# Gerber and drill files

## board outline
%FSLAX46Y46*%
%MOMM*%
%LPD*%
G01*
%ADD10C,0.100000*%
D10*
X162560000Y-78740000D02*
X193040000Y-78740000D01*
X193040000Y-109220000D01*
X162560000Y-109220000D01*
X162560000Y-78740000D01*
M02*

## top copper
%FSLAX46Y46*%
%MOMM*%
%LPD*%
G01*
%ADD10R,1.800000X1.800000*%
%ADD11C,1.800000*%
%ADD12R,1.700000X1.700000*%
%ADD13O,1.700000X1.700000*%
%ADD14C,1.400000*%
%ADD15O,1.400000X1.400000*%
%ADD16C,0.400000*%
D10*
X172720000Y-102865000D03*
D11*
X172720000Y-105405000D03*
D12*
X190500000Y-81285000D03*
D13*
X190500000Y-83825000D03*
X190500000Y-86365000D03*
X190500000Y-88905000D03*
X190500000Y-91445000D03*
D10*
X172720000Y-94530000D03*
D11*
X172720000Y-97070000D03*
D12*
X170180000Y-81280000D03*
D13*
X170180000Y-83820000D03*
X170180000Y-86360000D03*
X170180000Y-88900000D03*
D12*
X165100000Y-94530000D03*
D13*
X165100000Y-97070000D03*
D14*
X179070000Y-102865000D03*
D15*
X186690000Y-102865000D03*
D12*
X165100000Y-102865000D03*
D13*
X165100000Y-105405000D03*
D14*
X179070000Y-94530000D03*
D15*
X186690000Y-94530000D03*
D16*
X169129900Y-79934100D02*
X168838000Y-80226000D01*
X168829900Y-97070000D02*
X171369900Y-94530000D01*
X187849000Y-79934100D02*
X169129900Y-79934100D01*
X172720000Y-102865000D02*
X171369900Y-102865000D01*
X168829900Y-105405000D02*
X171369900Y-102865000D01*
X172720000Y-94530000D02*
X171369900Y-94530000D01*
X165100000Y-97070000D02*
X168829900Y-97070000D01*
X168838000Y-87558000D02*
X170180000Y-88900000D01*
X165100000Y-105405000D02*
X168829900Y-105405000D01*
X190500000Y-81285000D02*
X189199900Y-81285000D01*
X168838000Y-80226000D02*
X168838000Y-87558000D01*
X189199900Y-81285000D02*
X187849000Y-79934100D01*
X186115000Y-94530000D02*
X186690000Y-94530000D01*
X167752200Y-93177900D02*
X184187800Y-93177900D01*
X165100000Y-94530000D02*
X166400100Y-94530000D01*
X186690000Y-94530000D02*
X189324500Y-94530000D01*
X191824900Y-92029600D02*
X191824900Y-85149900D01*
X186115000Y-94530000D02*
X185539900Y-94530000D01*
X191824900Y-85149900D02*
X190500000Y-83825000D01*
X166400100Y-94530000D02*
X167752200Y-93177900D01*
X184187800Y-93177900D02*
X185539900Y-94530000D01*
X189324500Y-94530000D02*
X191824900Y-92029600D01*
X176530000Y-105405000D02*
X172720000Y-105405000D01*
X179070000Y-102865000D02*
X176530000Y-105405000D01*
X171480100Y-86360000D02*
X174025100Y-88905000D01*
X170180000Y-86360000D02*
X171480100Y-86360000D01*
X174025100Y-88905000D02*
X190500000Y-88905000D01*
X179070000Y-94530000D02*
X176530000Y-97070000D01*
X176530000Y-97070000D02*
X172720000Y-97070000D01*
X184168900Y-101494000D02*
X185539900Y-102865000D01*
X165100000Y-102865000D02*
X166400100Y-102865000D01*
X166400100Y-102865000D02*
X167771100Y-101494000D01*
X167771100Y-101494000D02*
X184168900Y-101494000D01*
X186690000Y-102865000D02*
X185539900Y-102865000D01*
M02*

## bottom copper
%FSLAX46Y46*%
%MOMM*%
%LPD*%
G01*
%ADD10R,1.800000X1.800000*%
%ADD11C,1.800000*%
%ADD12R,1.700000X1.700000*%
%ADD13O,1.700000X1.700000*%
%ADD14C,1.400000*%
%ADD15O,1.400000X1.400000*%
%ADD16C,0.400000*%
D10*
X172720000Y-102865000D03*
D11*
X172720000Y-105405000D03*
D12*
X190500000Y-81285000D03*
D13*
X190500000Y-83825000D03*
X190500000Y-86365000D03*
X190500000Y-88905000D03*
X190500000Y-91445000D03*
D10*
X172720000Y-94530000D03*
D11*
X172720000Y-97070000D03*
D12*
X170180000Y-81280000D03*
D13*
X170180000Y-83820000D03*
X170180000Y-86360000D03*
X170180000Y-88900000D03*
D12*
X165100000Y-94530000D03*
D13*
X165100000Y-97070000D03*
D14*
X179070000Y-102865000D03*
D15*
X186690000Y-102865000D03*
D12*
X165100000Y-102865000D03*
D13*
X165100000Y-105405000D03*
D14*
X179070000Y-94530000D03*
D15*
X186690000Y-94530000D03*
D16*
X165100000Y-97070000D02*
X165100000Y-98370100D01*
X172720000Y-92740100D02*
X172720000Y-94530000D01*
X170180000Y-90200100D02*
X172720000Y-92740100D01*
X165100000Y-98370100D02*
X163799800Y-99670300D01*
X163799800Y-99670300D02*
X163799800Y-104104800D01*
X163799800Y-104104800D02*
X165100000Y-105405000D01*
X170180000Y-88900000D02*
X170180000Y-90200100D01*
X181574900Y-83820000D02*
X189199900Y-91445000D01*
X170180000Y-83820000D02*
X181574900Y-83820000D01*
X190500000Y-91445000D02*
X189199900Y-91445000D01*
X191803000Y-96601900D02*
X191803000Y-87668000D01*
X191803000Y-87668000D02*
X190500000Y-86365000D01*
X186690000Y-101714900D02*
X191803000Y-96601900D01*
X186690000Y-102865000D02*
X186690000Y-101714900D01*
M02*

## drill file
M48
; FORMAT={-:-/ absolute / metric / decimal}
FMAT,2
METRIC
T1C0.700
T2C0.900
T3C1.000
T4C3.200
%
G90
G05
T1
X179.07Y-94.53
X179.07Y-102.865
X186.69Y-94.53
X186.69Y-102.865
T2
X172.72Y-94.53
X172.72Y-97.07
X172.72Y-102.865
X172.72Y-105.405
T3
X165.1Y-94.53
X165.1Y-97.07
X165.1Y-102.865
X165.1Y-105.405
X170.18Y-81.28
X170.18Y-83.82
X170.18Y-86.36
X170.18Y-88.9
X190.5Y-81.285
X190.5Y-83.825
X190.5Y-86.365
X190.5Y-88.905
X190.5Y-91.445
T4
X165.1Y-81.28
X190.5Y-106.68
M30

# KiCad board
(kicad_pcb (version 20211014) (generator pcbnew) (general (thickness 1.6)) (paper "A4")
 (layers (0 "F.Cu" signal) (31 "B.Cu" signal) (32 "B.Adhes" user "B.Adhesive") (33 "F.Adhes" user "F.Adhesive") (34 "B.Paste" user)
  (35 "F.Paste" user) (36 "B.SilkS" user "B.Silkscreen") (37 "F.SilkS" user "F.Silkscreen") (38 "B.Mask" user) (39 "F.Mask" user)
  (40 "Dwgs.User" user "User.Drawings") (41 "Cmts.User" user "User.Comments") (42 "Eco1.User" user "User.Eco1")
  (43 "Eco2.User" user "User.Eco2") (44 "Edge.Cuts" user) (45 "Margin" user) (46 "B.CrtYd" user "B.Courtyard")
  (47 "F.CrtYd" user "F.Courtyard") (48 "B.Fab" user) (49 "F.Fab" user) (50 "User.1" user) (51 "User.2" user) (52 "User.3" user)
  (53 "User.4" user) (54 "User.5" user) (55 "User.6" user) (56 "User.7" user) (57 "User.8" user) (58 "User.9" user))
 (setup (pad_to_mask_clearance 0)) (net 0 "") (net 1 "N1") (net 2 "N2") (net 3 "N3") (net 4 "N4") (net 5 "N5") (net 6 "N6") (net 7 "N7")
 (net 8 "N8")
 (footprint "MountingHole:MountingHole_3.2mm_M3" (layer "F.Cu") (at 190.5 106.68)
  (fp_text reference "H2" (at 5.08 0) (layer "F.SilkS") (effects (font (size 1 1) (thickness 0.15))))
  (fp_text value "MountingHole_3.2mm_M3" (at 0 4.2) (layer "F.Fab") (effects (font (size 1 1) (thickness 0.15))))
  (pad "" np_thru_hole circle (at 0 0) (size 3.2 3.2) (drill 3.2) (layers *.Cu *.Mask)))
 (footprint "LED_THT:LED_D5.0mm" (layer "F.Cu") (at 172.72 102.865 -90)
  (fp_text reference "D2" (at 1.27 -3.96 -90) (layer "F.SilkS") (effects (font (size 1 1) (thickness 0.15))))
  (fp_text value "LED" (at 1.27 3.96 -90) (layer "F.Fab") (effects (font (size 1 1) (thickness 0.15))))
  (pad "1" thru_hole rect (at 0 0 270) (size 1.8 1.8) (drill 0.9) (layers *.Cu *.Mask) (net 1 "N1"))
  (pad "2" thru_hole circle (at 2.54 0 270) (size 1.8 1.8) (drill 0.9) (layers *.Cu *.Mask) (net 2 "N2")))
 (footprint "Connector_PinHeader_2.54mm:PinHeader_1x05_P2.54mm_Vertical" (layer "F.Cu") (at 190.5 81.285)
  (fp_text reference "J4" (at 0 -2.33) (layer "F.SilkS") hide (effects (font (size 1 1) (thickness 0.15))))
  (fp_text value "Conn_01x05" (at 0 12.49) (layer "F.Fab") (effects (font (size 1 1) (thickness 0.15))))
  (pad "1" thru_hole rect (at 0 0) (size 1.7 1.7) (drill 1) (layers *.Cu *.Mask) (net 1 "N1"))
  (pad "2" thru_hole oval (at 0 2.54) (size 1.7 1.7) (drill 1) (layers *.Cu *.Mask) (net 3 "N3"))
  (pad "3" thru_hole oval (at 0 5.08) (size 1.7 1.7) (drill 1) (layers *.Cu *.Mask) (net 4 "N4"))
  (pad "4" thru_hole oval (at 0 7.62) (size 1.7 1.7) (drill 1) (layers *.Cu *.Mask) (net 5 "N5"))
  (pad "5" thru_hole oval (at 0 10.16) (size 1.7 1.7) (drill 1) (layers *.Cu *.Mask) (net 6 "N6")))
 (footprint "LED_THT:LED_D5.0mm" (layer "F.Cu") (at 172.72 94.53 -90)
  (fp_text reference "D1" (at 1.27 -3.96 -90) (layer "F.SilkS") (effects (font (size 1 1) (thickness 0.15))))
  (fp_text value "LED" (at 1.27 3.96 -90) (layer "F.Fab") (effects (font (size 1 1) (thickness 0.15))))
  (pad "1" thru_hole rect (at 0 0 270) (size 1.8 1.8) (drill 0.9) (layers *.Cu *.Mask) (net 1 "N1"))
  (pad "2" thru_hole circle (at 2.54 0 270) (size 1.8 1.8) (drill 0.9) (layers *.Cu *.Mask) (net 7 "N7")))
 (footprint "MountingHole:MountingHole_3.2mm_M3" (layer "F.Cu") (at 165.1 81.28)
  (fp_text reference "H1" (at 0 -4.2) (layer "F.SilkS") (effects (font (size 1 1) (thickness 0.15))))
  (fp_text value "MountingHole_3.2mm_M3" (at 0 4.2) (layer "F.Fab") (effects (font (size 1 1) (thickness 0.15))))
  (pad "" np_thru_hole circle (at 0 0) (size 3.2 3.2) (drill 3.2) (layers F&B.Cu *.Mask)))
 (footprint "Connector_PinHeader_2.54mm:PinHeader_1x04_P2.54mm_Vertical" (layer "F.Cu") (at 170.18 81.28)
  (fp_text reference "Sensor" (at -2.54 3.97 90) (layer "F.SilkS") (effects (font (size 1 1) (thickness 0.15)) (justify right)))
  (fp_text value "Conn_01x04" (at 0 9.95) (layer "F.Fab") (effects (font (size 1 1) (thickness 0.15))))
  (pad "1" thru_hole rect (at 0 0) (size 1.7 1.7) (drill 1) (layers *.Cu *.Mask) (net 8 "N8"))
  (pad "2" thru_hole oval (at 0 2.54) (size 1.7 1.7) (drill 1) (layers *.Cu *.Mask) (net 6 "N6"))
  (pad "3" thru_hole oval (at 0 5.08) (size 1.7 1.7) (drill 1) (layers *.Cu *.Mask) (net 5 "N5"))
  (pad "4" thru_hole oval (at 0 7.62) (size 1.7 1.7) (drill 1) (layers *.Cu *.Mask) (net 1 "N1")))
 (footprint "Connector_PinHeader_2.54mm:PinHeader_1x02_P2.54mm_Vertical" (layer "F.Cu") (at 165.1 94.53)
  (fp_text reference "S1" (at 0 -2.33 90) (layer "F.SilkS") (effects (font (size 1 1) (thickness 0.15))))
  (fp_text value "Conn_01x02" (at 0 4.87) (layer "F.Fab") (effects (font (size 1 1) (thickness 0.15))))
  (pad "1" thru_hole rect (at 0 0) (size 1.7 1.7) (drill 1) (layers *.Cu *.Mask) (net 3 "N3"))
  (pad "2" thru_hole oval (at 0 2.54) (size 1.7 1.7) (drill 1) (layers *.Cu *.Mask) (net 1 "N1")))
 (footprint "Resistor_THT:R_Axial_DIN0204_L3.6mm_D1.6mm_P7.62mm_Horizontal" (layer "F.Cu") (at 179.07 102.865)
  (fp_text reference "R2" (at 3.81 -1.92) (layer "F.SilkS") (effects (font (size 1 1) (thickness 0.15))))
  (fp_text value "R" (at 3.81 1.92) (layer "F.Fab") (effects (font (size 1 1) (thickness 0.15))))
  (pad "1" thru_hole circle (at 0 0) (size 1.4 1.4) (drill 0.7) (layers *.Cu *.Mask) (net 2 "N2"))
  (pad "2" thru_hole oval (at 7.62 0) (size 1.4 1.4) (drill 0.7) (layers *.Cu *.Mask) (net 4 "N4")))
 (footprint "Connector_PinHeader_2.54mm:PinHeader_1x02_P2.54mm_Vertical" (layer "F.Cu") (at 165.1 102.865)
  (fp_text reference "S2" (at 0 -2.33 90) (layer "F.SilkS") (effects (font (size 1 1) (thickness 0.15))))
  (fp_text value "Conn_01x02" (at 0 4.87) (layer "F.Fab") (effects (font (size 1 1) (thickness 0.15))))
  (pad "1" thru_hole rect (at 0 0) (size 1.7 1.7) (drill 1) (layers *.Cu *.Mask) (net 4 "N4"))
  (pad "2" thru_hole oval (at 0 2.54) (size 1.7 1.7) (drill 1) (layers *.Cu *.Mask) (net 1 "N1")))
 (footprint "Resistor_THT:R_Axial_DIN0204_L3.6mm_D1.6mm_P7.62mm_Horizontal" (layer "F.Cu") (at 179.07 94.53)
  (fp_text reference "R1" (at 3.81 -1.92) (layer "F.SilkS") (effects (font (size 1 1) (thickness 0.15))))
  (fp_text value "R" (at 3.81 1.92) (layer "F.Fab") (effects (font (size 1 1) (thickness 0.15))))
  (pad "1" thru_hole circle (at 0 0) (size 1.4 1.4) (drill 0.7) (layers *.Cu *.Mask) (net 7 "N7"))
  (pad "2" thru_hole oval (at 7.62 0) (size 1.4 1.4) (drill 0.7) (layers *.Cu *.Mask) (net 3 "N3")))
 (gr_rect (start 162.56 78.74) (end 193.04 109.22) (layer "Edge.Cuts") (width 0.1) (fill none))
 (segment (start 169.1299 79.9341) (end 168.838 80.226) (width 0.4) (layer "F.Cu") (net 1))
 (segment (start 168.8299 97.07) (end 171.3699 94.53) (width 0.4) (layer "F.Cu") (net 1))
 (segment (start 187.849 79.9341) (end 169.1299 79.9341) (width 0.4) (layer "F.Cu") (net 1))
 (segment (start 172.72 102.865) (end 171.3699 102.865) (width 0.4) (layer "F.Cu") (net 1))
 (segment (start 168.8299 105.405) (end 171.3699 102.865) (width 0.4) (layer "F.Cu") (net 1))
 (segment (start 172.72 94.53) (end 171.3699 94.53) (width 0.4) (layer "F.Cu") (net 1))
 (segment (start 165.1 97.07) (end 168.8299 97.07) (width 0.4) (layer "F.Cu") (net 1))
 (segment (start 168.838 87.558) (end 170.18 88.9) (width 0.4) (layer "F.Cu") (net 1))
 (segment (start 165.1 105.405) (end 168.8299 105.405) (width 0.4) (layer "F.Cu") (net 1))
 (segment (start 190.5 81.285) (end 189.1999 81.285) (width 0.4) (layer "F.Cu") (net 1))
 (segment (start 168.838 80.226) (end 168.838 87.558) (width 0.4) (layer "F.Cu") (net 1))
 (segment (start 189.1999 81.285) (end 187.849 79.9341) (width 0.4) (layer "F.Cu") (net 1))
 (segment (start 165.1 97.07) (end 165.1 98.3701) (width 0.4) (layer "B.Cu") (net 1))
 (segment (start 172.72 92.7401) (end 172.72 94.53) (width 0.4) (layer "B.Cu") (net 1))
 (segment (start 170.18 90.2001) (end 172.72 92.7401) (width 0.4) (layer "B.Cu") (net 1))
 (segment (start 165.1 98.3701) (end 163.7998 99.6703) (width 0.4) (layer "B.Cu") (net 1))
 (segment (start 163.7998 99.6703) (end 163.7998 104.1048) (width 0.4) (layer "B.Cu") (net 1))
 (segment (start 163.7998 104.1048) (end 165.1 105.405) (width 0.4) (layer "B.Cu") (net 1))
 (segment (start 170.18 88.9) (end 170.18 90.2001) (width 0.4) (layer "B.Cu") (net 1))
 (segment (start 186.115 94.53) (end 186.69 94.53) (width 0.4) (layer "F.Cu") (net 3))
 (segment (start 167.7522 93.1779) (end 184.1878 93.1779) (width 0.4) (layer "F.Cu") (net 3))
 (segment (start 165.1 94.53) (end 166.4001 94.53) (width 0.4) (layer "F.Cu") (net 3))
 (segment (start 186.69 94.53) (end 189.3245 94.53) (width 0.4) (layer "F.Cu") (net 3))
 (segment (start 191.8249 92.0296) (end 191.8249 85.1499) (width 0.4) (layer "F.Cu") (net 3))
 (segment (start 186.115 94.53) (end 185.5399 94.53) (width 0.4) (layer "F.Cu") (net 3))
 (segment (start 191.8249 85.1499) (end 190.5 83.825) (width 0.4) (layer "F.Cu") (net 3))
 (segment (start 166.4001 94.53) (end 167.7522 93.1779) (width 0.4) (layer "F.Cu") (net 3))
 (segment (start 184.1878 93.1779) (end 185.5399 94.53) (width 0.4) (layer "F.Cu") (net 3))
 (segment (start 189.3245 94.53) (end 191.8249 92.0296) (width 0.4) (layer "F.Cu") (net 3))
 (segment (start 176.53 105.405) (end 172.72 105.405) (width 0.4) (layer "F.Cu") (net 2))
 (segment (start 179.07 102.865) (end 176.53 105.405) (width 0.4) (layer "F.Cu") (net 2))
 (segment (start 181.5749 83.82) (end 189.1999 91.445) (width 0.4) (layer "B.Cu") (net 6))
 (segment (start 170.18 83.82) (end 181.5749 83.82) (width 0.4) (layer "B.Cu") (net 6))
 (segment (start 190.5 91.445) (end 189.1999 91.445) (width 0.4) (layer "B.Cu") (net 6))
 (segment (start 171.4801 86.36) (end 174.0251 88.905) (width 0.4) (layer "F.Cu") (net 5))
 (segment (start 170.18 86.36) (end 171.4801 86.36) (width 0.4) (layer "F.Cu") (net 5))
 (segment (start 174.0251 88.905) (end 190.5 88.905) (width 0.4) (layer "F.Cu") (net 5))
 (segment (start 179.07 94.53) (end 176.53 97.07) (width 0.4) (layer "F.Cu") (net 7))
 (segment (start 176.53 97.07) (end 172.72 97.07) (width 0.4) (layer "F.Cu") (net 7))
 (segment (start 184.1689 101.494) (end 185.5399 102.865) (width 0.4) (layer "F.Cu") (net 4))
 (segment (start 165.1 102.865) (end 166.4001 102.865) (width 0.4) (layer "F.Cu") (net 4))
 (segment (start 166.4001 102.865) (end 167.7711 101.494) (width 0.4) (layer "F.Cu") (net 4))
 (segment (start 167.7711 101.494) (end 184.1689 101.494) (width 0.4) (layer "F.Cu") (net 4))
 (segment (start 186.69 102.865) (end 185.5399 102.865) (width 0.4) (layer "F.Cu") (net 4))
 (segment (start 191.803 96.6019) (end 191.803 87.668) (width 0.4) (layer "B.Cu") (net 4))
 (segment (start 191.803 87.668) (end 190.5 86.365) (width 0.4) (layer "B.Cu") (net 4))
 (segment (start 186.69 101.7149) (end 191.803 96.6019) (width 0.4) (layer "B.Cu") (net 4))
 (segment (start 186.69 102.865) (end 186.69 101.7149) (width 0.4) (layer "B.Cu") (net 4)))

